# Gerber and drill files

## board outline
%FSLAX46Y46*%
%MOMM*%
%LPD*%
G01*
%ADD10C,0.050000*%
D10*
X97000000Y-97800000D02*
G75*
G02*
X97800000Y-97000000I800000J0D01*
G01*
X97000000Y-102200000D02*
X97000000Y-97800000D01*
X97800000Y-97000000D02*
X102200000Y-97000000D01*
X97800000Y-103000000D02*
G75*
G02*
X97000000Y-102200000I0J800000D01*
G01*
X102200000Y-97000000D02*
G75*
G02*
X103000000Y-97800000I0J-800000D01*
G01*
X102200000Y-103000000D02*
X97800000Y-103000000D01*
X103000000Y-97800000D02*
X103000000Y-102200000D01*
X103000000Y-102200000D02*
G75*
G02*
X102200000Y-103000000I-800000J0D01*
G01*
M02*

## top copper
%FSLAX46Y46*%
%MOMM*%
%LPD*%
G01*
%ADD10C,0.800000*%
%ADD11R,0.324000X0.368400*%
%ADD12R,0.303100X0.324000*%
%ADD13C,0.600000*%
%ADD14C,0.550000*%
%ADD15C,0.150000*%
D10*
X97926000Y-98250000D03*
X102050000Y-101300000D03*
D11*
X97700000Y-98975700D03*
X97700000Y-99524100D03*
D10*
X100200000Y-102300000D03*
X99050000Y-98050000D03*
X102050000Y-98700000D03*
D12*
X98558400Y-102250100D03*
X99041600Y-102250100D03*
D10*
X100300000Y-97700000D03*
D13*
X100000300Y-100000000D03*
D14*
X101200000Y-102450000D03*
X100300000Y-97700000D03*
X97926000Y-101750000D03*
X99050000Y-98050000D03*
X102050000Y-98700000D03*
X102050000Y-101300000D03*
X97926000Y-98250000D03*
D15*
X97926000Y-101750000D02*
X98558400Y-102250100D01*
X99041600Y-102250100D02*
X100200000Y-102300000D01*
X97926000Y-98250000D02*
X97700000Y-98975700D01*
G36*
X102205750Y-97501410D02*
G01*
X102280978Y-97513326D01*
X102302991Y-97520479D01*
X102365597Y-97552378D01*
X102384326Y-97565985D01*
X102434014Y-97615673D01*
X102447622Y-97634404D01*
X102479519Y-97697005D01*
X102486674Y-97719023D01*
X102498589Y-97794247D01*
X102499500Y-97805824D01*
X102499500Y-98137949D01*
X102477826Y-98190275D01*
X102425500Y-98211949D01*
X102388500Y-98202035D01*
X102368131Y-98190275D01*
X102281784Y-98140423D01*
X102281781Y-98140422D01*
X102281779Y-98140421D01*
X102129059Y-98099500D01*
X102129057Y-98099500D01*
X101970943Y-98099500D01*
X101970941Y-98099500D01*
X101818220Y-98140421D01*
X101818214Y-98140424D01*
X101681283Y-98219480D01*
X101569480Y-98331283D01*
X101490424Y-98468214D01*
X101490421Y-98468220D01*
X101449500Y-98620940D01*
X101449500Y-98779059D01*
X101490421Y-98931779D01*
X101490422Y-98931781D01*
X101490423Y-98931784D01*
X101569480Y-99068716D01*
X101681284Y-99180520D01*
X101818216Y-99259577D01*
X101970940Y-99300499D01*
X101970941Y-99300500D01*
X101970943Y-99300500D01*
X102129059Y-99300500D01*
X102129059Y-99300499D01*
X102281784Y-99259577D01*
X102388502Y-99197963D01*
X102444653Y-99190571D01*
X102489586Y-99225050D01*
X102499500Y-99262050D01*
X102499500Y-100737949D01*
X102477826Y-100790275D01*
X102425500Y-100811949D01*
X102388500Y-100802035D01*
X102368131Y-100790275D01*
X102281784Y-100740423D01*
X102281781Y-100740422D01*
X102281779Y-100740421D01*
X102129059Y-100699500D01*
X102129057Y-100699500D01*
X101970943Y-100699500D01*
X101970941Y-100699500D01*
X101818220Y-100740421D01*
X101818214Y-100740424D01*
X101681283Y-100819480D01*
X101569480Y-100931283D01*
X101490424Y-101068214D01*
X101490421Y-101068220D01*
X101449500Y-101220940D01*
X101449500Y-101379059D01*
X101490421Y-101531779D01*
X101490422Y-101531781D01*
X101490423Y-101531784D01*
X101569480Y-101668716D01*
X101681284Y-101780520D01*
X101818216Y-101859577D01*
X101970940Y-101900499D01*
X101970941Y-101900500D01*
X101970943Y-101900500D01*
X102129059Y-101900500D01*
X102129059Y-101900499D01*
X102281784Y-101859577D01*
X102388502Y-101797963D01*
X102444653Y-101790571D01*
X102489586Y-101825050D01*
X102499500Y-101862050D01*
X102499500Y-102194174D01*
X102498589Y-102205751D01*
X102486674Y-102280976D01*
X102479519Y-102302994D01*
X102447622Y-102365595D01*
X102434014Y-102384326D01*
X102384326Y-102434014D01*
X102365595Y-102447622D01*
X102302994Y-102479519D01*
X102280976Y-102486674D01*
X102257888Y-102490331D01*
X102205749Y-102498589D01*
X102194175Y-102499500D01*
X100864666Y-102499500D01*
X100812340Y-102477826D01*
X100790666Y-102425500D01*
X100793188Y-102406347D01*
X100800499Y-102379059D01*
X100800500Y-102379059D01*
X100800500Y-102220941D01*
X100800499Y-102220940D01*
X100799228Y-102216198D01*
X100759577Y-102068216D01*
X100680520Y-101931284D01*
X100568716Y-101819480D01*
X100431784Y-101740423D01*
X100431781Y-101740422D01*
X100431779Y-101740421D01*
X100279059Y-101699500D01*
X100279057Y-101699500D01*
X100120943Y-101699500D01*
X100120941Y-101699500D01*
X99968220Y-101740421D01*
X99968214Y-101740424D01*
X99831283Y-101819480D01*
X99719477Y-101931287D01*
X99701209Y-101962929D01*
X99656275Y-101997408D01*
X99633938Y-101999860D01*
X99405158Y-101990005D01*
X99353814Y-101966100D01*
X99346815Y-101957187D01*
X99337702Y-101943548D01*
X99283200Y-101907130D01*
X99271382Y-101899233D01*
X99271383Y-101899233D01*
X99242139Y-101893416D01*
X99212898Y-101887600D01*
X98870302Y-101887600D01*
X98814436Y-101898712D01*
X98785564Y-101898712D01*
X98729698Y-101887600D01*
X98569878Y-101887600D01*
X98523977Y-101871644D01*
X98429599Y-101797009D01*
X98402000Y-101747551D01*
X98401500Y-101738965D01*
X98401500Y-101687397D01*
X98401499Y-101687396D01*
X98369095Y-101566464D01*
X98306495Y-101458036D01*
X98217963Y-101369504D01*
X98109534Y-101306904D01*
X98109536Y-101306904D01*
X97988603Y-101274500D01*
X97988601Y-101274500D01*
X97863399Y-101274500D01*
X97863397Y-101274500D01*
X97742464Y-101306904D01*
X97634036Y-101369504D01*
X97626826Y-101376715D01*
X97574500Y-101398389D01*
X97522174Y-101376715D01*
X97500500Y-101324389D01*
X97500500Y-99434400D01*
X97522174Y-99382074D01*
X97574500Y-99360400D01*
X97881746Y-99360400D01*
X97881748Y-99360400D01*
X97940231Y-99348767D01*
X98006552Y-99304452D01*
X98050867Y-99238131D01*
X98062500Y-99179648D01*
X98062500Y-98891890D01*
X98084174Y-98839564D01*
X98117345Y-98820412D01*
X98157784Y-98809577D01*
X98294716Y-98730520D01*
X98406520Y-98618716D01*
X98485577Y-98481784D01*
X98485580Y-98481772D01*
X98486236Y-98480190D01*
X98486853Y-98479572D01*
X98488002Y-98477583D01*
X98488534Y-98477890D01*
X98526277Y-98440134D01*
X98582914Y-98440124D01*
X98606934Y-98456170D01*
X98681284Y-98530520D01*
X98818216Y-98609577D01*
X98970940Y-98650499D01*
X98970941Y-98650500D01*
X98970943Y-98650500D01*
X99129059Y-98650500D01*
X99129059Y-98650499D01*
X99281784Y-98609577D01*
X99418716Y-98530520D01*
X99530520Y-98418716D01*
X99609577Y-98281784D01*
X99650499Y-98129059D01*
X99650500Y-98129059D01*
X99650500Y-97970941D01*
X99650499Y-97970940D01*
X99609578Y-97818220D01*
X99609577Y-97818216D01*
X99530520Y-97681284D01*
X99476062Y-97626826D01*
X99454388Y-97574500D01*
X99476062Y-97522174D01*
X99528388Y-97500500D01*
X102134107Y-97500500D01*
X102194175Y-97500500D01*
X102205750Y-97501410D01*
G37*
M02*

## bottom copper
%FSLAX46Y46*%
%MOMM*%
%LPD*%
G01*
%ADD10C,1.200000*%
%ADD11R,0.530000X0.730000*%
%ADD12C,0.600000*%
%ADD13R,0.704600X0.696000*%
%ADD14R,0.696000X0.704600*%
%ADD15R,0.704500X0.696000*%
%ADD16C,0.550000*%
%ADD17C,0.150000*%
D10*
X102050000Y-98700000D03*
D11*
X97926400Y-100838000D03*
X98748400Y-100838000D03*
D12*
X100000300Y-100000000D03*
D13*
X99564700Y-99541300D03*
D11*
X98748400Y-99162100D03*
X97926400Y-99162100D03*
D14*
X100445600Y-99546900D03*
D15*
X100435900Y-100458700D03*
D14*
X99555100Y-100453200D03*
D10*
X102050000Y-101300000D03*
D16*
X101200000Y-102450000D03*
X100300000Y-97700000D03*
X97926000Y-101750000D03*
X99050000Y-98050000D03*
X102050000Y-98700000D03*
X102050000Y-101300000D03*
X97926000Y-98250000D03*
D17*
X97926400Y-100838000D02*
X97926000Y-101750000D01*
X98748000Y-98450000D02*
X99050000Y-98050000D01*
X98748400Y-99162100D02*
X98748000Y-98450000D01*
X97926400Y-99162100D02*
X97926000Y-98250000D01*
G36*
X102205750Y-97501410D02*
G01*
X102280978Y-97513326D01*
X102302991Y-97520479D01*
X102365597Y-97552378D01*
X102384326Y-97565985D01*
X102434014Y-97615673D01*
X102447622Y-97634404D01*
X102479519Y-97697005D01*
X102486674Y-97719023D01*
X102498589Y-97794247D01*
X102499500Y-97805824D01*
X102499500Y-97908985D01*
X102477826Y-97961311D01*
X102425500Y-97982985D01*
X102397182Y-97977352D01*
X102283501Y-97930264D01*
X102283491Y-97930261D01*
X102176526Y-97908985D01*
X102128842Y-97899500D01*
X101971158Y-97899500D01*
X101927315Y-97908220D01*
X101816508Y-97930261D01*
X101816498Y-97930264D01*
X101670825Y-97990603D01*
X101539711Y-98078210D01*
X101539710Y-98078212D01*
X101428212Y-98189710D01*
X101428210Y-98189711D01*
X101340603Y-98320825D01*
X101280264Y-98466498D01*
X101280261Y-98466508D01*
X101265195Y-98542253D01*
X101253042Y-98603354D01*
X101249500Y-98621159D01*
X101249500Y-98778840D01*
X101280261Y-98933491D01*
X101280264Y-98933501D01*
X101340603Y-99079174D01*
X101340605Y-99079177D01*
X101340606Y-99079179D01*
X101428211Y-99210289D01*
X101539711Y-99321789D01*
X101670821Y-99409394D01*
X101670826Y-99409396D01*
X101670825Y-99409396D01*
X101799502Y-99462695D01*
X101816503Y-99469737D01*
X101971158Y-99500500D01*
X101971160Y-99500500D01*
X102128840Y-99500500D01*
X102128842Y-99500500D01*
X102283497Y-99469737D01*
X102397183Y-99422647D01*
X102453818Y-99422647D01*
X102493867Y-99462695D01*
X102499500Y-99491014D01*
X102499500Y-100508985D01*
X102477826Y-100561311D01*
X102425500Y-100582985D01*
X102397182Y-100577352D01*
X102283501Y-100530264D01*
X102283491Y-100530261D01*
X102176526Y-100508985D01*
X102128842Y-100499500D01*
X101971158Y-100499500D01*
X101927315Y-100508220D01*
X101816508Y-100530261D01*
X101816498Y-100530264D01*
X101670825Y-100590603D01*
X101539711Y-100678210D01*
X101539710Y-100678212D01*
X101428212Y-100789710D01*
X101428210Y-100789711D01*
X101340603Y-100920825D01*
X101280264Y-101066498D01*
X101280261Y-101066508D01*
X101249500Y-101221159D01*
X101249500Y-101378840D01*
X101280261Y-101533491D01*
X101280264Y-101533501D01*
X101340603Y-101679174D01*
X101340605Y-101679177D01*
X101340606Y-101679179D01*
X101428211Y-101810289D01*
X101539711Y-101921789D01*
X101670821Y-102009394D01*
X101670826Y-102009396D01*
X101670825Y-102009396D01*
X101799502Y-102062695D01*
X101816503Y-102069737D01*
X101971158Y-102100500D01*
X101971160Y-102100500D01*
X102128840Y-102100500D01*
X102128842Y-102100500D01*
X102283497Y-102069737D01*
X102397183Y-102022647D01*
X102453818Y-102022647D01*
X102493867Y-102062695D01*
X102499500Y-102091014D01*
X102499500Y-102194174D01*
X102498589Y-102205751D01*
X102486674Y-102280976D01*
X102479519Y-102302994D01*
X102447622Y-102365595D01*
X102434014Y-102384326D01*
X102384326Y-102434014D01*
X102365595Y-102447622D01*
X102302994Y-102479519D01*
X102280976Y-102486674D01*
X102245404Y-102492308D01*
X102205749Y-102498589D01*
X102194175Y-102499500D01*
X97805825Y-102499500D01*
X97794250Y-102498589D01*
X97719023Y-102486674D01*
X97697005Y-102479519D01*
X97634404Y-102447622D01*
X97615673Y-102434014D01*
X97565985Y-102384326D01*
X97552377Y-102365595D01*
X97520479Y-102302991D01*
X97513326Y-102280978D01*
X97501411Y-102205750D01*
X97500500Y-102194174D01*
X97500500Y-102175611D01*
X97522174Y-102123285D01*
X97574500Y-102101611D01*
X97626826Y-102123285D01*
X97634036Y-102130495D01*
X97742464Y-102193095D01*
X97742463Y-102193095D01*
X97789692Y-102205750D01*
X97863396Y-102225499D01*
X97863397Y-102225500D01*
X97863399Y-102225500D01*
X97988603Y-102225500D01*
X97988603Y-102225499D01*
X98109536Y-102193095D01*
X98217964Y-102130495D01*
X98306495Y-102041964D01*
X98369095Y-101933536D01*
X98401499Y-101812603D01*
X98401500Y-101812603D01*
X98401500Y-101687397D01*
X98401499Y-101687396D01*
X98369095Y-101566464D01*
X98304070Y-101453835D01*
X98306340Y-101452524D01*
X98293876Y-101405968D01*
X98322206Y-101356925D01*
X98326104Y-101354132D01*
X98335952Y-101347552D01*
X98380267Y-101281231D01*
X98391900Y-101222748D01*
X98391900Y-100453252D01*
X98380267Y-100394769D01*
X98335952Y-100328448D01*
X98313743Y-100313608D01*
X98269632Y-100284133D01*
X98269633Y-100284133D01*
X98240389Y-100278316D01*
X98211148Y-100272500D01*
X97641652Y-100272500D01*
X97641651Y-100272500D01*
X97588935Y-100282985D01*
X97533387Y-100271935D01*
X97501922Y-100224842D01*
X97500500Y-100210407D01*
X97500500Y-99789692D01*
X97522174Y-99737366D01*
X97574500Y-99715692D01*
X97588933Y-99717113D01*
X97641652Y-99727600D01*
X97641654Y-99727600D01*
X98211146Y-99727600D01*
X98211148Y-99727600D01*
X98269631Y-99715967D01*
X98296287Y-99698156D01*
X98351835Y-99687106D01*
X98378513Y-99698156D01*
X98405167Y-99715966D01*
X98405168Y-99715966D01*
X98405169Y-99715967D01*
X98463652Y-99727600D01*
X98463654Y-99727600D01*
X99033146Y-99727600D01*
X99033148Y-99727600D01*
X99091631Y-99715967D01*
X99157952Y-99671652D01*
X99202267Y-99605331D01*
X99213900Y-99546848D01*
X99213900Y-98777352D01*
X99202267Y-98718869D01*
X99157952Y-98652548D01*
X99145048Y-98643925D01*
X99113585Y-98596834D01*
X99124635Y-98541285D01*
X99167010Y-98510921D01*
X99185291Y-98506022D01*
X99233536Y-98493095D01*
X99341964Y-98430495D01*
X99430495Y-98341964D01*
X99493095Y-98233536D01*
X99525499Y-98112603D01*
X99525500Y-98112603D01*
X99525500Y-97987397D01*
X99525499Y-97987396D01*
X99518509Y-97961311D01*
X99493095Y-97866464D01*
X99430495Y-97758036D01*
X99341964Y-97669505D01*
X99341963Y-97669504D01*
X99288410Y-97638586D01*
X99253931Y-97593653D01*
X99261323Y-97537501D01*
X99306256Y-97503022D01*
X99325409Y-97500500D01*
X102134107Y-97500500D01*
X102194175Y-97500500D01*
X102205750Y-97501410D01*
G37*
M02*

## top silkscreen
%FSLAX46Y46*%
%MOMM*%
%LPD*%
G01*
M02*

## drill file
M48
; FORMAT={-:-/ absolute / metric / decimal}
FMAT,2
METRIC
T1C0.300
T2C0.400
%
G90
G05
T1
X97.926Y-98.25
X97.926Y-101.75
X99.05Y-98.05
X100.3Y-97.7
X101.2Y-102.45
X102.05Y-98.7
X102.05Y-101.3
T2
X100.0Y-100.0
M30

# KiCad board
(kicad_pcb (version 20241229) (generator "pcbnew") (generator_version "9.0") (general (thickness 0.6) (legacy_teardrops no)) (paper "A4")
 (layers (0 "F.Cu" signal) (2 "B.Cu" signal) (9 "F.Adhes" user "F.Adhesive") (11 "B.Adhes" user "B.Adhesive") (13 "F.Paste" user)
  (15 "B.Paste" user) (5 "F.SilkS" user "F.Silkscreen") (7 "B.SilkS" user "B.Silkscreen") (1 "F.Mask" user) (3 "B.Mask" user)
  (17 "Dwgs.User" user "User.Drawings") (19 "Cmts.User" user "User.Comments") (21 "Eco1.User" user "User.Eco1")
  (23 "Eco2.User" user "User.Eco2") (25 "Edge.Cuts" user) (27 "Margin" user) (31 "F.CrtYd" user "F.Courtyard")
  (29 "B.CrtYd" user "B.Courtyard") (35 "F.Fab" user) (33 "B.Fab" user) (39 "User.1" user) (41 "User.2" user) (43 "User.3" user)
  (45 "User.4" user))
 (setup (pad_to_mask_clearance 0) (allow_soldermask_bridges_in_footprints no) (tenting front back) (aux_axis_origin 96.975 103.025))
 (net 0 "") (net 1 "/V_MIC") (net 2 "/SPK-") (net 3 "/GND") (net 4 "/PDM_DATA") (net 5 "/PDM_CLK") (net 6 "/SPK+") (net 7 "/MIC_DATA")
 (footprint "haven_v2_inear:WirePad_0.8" (layer "F.Cu") (at 97.926 98.25)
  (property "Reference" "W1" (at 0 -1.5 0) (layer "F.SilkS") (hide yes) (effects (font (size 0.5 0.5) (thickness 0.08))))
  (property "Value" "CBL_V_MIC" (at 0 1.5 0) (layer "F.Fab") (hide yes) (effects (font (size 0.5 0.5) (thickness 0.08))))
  (pad "1" smd circle (at 0 0) (size 0.8 0.8) (layers "F.Cu" "F.Mask") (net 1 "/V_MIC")))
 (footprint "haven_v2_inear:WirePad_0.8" (layer "F.Cu") (at 102.05 101.3)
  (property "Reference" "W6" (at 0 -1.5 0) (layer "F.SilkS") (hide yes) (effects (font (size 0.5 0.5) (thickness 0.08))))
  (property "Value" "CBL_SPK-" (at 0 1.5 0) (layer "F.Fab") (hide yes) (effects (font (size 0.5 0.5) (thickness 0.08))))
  (pad "1" smd circle (at 0 0) (size 0.8 0.8) (layers "F.Cu" "F.Mask") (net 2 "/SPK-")))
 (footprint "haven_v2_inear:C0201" (layer "F.Cu") (at 97.7 99.25 -90)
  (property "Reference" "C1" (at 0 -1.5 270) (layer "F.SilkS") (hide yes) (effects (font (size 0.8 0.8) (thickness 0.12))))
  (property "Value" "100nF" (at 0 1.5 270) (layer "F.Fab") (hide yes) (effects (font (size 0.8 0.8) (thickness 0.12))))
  (pad "1" smd rect (at -0.2743 0 270) (size 0.3684 0.324) (layers "F.Cu" "F.Mask" "F.Paste") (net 1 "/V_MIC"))
  (pad "2" smd rect (at 0.2741 0 270) (size 0.3684 0.324) (layers "F.Cu" "F.Mask" "F.Paste") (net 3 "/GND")))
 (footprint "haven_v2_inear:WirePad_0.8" (layer "F.Cu") (at 100.2 102.3)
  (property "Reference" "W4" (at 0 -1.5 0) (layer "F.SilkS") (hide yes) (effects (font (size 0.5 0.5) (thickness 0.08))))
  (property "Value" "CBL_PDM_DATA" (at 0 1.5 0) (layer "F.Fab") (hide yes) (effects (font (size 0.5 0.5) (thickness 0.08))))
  (pad "1" smd circle (at 0 0) (size 0.8 0.8) (layers "F.Cu" "F.Mask") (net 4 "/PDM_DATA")))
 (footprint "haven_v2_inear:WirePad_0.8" (layer "F.Cu") (at 99.05 98.05)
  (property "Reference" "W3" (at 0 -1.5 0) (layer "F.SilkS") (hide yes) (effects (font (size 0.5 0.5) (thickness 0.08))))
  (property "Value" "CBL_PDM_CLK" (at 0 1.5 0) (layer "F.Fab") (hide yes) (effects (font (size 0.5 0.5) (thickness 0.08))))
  (pad "1" smd circle (at 0 0) (size 0.8 0.8) (layers "F.Cu" "F.Mask") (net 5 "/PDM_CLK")))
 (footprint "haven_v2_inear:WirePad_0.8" (layer "F.Cu") (at 102.05 98.7)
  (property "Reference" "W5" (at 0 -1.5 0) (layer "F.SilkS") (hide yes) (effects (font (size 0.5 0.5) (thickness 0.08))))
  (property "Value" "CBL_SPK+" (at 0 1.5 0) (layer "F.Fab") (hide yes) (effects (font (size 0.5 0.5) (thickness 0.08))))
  (pad "1" smd circle (at 0 0) (size 0.8 0.8) (layers "F.Cu" "F.Mask") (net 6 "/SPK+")))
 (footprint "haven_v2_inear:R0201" (layer "F.Cu") (at 98.8 102.25)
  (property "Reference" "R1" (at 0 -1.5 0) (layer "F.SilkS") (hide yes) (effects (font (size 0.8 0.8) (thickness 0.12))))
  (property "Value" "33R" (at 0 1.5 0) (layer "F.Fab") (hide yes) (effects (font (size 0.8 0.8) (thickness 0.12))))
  (pad "1" smd rect (at -0.2416 0.0001) (size 0.3031 0.324) (layers "F.Cu" "F.Mask" "F.Paste") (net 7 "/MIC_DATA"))
  (pad "2" smd rect (at 0.2416 0.0001) (size 0.3031 0.324) (layers "F.Cu" "F.Mask" "F.Paste") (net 4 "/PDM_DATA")))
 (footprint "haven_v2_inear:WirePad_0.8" (layer "F.Cu") (at 100.3 97.7)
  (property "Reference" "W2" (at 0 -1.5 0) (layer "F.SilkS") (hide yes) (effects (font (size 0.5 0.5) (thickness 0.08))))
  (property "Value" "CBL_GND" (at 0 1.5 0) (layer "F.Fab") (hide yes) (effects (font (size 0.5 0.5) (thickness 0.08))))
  (pad "1" smd circle (at 0 0) (size 0.8 0.8) (layers "F.Cu" "F.Mask") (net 3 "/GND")))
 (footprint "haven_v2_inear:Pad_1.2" (layer "B.Cu") (at 102.05 98.7)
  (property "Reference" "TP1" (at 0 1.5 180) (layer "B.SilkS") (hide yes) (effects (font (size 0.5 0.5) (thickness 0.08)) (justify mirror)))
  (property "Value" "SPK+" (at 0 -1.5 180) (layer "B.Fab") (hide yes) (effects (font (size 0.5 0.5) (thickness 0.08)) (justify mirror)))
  (pad "1" smd circle (at 0 0) (size 1.2 1.2) (layers "B.Cu" "B.Mask") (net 6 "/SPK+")))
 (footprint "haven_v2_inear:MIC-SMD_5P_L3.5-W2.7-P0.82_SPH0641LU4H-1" (layer "B.Cu") (at 99.186 100 90)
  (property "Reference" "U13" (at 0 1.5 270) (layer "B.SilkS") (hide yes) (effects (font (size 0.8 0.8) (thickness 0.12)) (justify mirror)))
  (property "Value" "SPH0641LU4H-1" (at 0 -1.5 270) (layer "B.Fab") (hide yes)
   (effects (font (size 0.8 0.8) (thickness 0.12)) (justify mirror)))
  (pad "1" smd rect (at -0.838 -1.2596 270) (size 0.73 0.53) (layers "B.Cu" "B.Mask" "B.Paste") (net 7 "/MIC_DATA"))
  (pad "2" smd rect (at -0.838 -0.4376 270) (size 0.73 0.53) (layers "B.Cu" "B.Mask" "B.Paste") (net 3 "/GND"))
  (pad "3" thru_hole circle (at 0 0.8143 90) (size 0.6 0.6) (drill 0.4) (layers "*.Cu" "*.Mask") (remove_unused_layers no) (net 3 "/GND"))
  (pad "3" smd rect (at 0.4587 0.3787 90) (size 0.696 0.7046) (layers "B.Cu" "B.Mask" "B.Paste") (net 3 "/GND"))
  (pad "4" smd rect (at 0.8379 -0.4376 270) (size 0.73 0.53) (layers "B.Cu" "B.Mask" "B.Paste") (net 5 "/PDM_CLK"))
  (pad "5" smd rect (at 0.8379 -1.2596 270) (size 0.73 0.53) (layers "B.Cu" "B.Mask" "B.Paste") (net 1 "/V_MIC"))
  (pad "6" smd rect (at 0.4531 1.2596 90) (size 0.7046 0.696) (layers "B.Cu" "B.Mask" "B.Paste") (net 3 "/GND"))
  (pad "7" smd rect (at -0.4587 1.2499 90) (size 0.696 0.7045) (layers "B.Cu" "B.Mask" "B.Paste") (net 3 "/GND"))
  (pad "8" smd rect (at -0.4532 0.3691 90) (size 0.7046 0.696) (layers "B.Cu" "B.Mask" "B.Paste") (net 3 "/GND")))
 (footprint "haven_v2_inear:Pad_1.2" (layer "B.Cu") (at 102.05 101.3)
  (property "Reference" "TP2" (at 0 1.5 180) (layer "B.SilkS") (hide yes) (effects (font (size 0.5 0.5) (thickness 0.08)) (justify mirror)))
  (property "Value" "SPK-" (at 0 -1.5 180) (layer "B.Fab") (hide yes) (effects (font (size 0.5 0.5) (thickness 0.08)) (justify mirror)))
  (pad "1" smd circle (at 0 0) (size 1.2 1.2) (layers "B.Cu" "B.Mask") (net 2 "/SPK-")))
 (gr_arc (start 97 97.8) (mid 97.234315 97.234315) (end 97.8 97) (stroke (width 0.05) (type default)) (layer "Edge.Cuts"))
 (gr_line (start 97 102.2) (end 97 97.8) (stroke (width 0.05) (type default)) (layer "Edge.Cuts"))
 (gr_line (start 97.8 97) (end 102.2 97) (stroke (width 0.05) (type default)) (layer "Edge.Cuts"))
 (gr_arc (start 97.8 103) (mid 97.234315 102.765685) (end 97 102.2) (stroke (width 0.05) (type default)) (layer "Edge.Cuts"))
 (gr_arc (start 102.2 97) (mid 102.765685 97.234315) (end 103 97.8) (stroke (width 0.05) (type default)) (layer "Edge.Cuts"))
 (gr_line (start 102.2 103) (end 97.8 103) (stroke (width 0.05) (type default)) (layer "Edge.Cuts"))
 (gr_line (start 103 97.8) (end 103 102.2) (stroke (width 0.05) (type default)) (layer "Edge.Cuts"))
 (gr_arc (start 103 102.2) (mid 102.765685 102.765685) (end 102.2 103) (stroke (width 0.05) (type default)) (layer "Edge.Cuts"))
 (via (at 101.2 102.45) (size 0.55) (drill 0.3) (layers "F.Cu" "B.Cu") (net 3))
 (via (at 100.3 97.7) (size 0.55) (drill 0.3) (layers "F.Cu" "B.Cu") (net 3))
 (segment (start 97.926 101.75) (end 98.5584 102.2501) (width 0.15) (layer "F.Cu") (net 7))
 (via (at 97.926 101.75) (size 0.55) (drill 0.3) (layers "F.Cu" "B.Cu") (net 7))
 (segment (start 97.9264 100.838) (end 97.926 101.75) (width 0.15) (layer "B.Cu") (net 7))
 (via (at 99.05 98.05) (size 0.55) (drill 0.3) (layers "F.Cu" "B.Cu") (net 5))
 (segment (start 98.748 98.45) (end 99.05 98.05) (width 0.15) (layer "B.Cu") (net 5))
 (segment (start 98.7484 99.1621) (end 98.748 98.45) (width 0.15) (layer "B.Cu") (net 5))
 (segment (start 99.0416 102.2501) (end 100.2 102.3) (width 0.15) (layer "F.Cu") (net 4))
 (via (at 102.05 98.7) (size 0.55) (drill 0.3) (layers "F.Cu" "B.Cu") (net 6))
 (via (at 102.05 101.3) (size 0.55) (drill 0.3) (layers "F.Cu" "B.Cu") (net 2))
 (segment (start 97.926 98.25) (end 97.7 98.9757) (width 0.15) (layer "F.Cu") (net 1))
 (via (at 97.926 98.25) (size 0.55) (drill 0.3) (layers "F.Cu" "B.Cu") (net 1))
 (segment (start 97.9264 99.1621) (end 97.926 98.25) (width 0.15) (layer "B.Cu") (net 1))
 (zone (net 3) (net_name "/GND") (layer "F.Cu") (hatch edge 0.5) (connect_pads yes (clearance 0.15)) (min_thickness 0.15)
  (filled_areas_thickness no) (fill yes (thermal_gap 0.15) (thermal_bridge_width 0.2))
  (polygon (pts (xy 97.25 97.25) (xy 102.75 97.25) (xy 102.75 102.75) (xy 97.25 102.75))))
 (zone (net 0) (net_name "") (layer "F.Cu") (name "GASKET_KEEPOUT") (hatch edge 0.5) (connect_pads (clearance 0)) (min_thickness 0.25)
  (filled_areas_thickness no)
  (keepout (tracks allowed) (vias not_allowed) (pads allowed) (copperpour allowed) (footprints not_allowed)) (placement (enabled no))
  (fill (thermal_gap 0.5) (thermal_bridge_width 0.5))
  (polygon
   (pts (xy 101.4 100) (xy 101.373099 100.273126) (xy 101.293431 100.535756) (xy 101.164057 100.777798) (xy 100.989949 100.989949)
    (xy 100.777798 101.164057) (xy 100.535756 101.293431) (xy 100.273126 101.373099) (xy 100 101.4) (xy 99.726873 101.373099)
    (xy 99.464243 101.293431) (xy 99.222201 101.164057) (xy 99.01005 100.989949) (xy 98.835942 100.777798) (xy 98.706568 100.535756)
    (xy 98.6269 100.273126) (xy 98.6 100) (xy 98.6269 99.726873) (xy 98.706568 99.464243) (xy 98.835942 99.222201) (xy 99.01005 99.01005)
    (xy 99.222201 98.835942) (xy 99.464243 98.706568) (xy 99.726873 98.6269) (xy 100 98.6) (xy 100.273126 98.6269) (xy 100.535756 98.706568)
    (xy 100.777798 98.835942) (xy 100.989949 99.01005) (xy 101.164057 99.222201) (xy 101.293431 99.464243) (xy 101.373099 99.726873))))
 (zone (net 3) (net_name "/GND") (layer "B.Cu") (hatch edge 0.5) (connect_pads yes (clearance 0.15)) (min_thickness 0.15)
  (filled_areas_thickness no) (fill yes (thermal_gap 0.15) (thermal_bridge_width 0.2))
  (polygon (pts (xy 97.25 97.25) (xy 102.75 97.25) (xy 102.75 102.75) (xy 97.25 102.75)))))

